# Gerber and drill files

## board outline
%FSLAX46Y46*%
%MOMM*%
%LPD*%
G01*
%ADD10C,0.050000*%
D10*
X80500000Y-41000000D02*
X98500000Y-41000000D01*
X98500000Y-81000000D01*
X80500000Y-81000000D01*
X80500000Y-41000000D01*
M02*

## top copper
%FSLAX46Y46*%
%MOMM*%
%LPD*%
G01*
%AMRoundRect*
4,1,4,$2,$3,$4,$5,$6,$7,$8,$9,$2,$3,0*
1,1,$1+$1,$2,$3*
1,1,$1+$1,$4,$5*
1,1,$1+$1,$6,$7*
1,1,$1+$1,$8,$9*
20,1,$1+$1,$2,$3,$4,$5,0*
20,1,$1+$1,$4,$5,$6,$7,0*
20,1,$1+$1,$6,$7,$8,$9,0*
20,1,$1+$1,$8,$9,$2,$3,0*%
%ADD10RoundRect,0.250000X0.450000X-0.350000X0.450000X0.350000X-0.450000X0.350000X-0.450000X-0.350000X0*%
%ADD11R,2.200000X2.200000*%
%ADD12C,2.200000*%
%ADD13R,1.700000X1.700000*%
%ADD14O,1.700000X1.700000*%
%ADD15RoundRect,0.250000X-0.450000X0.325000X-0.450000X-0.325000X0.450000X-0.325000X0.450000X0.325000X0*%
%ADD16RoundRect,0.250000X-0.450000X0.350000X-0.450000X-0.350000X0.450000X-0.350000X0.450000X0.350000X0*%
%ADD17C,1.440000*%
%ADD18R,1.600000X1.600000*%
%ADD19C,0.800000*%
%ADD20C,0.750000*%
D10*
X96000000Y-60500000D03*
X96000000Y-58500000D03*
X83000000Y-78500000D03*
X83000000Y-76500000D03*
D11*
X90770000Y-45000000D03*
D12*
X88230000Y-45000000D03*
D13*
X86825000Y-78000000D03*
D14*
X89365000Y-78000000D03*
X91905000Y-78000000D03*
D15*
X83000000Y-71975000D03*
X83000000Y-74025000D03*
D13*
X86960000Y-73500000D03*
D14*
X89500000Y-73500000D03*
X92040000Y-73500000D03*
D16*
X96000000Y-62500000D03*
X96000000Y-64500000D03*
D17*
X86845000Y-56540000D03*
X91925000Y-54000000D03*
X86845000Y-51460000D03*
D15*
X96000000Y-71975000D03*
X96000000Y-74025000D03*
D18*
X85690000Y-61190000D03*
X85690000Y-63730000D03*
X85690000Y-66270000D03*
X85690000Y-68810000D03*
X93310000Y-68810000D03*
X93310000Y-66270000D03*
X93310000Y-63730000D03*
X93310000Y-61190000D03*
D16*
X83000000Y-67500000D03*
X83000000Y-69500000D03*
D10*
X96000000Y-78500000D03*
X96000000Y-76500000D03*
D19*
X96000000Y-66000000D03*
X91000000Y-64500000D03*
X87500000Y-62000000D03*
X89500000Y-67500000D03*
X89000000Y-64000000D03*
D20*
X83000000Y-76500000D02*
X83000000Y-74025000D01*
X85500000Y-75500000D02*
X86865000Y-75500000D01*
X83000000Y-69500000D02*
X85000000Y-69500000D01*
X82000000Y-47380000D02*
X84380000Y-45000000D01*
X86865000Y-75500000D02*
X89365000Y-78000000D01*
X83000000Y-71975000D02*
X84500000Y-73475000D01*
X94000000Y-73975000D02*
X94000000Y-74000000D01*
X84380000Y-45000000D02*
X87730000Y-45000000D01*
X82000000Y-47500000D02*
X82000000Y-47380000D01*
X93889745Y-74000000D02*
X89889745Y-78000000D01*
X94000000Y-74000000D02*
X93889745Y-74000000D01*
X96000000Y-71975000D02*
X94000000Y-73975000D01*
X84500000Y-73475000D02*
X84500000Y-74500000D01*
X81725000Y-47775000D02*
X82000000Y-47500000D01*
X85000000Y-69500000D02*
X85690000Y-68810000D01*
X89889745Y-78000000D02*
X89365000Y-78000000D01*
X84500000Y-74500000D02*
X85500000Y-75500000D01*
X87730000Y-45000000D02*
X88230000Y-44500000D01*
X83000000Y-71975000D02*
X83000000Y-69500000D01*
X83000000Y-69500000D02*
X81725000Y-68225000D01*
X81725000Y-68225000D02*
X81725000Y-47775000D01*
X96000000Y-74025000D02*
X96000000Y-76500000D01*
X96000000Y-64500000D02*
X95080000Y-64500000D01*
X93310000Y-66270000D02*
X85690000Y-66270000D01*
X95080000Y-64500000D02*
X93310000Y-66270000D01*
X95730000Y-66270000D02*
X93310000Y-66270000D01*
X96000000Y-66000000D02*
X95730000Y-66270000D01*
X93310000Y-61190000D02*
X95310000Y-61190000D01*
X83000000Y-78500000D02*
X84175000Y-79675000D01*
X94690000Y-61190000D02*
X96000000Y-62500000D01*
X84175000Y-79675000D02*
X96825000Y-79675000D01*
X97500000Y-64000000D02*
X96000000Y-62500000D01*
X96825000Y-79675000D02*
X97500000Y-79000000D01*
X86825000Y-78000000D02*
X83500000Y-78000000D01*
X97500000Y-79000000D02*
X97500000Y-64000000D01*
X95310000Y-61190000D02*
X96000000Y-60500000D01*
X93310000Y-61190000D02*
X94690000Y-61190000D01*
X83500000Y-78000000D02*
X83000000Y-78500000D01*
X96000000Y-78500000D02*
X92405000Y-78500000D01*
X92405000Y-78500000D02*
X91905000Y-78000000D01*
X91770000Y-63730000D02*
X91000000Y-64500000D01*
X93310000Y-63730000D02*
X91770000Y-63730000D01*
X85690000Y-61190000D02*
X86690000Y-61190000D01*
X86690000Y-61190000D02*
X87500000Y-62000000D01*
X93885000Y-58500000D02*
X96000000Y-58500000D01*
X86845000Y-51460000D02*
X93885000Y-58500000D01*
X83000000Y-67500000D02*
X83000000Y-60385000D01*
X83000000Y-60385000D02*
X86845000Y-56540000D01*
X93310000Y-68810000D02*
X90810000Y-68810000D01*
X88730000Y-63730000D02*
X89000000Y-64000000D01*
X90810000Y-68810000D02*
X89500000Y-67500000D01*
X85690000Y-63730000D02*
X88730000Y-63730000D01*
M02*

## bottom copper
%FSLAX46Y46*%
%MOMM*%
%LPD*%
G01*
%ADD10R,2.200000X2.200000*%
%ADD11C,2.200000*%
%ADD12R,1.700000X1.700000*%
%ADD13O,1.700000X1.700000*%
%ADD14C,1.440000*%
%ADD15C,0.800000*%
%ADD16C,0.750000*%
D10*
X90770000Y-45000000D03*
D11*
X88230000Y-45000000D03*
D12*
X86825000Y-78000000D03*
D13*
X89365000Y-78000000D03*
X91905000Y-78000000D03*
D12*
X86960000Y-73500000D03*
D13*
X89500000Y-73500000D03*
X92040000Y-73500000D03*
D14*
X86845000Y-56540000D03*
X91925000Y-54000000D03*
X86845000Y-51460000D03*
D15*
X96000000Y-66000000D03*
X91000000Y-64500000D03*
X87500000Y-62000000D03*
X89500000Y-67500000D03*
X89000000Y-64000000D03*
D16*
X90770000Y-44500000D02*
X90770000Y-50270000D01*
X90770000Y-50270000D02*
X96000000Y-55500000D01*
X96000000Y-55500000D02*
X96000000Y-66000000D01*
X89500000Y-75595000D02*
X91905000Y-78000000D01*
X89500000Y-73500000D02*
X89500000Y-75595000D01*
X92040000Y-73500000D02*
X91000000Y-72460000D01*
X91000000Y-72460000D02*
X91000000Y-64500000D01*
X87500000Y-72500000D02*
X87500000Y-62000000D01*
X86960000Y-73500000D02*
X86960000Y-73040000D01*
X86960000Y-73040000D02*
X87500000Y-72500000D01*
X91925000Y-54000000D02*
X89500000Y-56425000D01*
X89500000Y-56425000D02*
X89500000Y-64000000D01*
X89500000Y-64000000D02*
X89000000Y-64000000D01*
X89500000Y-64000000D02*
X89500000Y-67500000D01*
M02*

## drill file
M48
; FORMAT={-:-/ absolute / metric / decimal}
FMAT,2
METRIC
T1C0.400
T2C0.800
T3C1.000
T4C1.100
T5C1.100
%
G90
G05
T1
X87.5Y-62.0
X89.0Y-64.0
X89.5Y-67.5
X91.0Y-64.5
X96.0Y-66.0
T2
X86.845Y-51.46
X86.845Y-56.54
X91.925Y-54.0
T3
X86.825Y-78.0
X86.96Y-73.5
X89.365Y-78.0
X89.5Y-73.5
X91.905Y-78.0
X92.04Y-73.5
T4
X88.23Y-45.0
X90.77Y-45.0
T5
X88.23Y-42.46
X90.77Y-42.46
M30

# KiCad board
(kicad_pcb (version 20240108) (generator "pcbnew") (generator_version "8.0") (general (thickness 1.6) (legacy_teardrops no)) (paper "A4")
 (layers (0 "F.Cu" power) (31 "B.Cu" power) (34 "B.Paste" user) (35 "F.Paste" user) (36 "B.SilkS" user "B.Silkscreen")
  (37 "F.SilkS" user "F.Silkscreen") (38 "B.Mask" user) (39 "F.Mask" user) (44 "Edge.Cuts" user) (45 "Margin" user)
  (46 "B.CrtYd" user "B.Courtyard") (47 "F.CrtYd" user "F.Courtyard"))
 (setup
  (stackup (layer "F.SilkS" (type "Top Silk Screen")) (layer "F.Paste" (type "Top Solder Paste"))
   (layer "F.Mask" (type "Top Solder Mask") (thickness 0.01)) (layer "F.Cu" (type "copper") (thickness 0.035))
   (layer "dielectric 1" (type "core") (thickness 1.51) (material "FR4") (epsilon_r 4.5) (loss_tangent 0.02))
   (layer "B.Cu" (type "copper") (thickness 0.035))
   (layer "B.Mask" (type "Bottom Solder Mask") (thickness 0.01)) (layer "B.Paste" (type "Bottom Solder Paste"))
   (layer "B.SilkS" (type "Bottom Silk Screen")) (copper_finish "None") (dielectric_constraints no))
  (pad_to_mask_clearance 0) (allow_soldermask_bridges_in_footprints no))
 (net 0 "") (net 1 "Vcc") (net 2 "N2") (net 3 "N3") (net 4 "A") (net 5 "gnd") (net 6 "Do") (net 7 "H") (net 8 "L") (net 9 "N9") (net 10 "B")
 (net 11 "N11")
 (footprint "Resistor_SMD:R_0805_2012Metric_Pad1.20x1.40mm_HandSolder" (layer "F.Cu") (at 96 59.5 90)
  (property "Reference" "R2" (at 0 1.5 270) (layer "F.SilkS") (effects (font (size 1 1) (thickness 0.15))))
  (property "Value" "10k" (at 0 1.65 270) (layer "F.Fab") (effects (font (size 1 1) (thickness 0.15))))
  (pad "1" smd roundrect (at -1 0 90) (size 1.2 1.4) (layers "F.Cu" "F.Paste" "F.Mask") (roundrect_rratio 0.208333) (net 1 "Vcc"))
  (pad "2" smd roundrect (at 1 0 90) (size 1.2 1.4) (layers "F.Cu" "F.Paste" "F.Mask") (roundrect_rratio 0.208333) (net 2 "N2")))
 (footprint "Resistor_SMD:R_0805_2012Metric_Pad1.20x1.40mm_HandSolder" (layer "F.Cu") (at 83 77.5 90)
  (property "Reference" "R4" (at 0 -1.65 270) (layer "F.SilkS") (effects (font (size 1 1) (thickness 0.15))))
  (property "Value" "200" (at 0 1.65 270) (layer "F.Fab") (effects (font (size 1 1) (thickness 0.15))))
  (pad "1" smd roundrect (at -1 0 90) (size 1.2 1.4) (layers "F.Cu" "F.Paste" "F.Mask") (roundrect_rratio 0.208333) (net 1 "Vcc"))
  (pad "2" smd roundrect (at 1 0 90) (size 1.2 1.4) (layers "F.Cu" "F.Paste" "F.Mask") (roundrect_rratio 0.208333) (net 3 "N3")))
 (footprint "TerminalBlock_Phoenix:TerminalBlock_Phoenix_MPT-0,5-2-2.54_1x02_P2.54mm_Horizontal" (layer "F.Cu") (at 90.77 45 180)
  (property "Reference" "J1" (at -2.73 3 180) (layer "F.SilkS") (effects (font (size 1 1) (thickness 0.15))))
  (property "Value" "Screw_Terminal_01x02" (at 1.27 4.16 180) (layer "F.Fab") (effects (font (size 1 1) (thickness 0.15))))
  (pad "" np_thru_hole circle (at 0 2.54 180) (size 1.1 1.1) (drill 1.1) (layers "*.Cu" "*.Mask"))
  (pad "" np_thru_hole circle (at 2.54 2.54 180) (size 1.1 1.1) (drill 1.1) (layers "*.Cu" "*.Mask"))
  (pad "1" thru_hole rect (at 0 0 180) (size 2.2 2.2) (drill 1.1) (layers "*.Cu" "*.Mask") (remove_unused_layers no) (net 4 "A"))
  (pad "2" thru_hole circle (at 2.54 0 180) (size 2.2 2.2) (drill 1.1) (layers "*.Cu" "*.Mask") (remove_unused_layers no) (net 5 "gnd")))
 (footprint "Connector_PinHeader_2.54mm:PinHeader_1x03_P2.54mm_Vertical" (layer "F.Cu") (at 86.825 78 90)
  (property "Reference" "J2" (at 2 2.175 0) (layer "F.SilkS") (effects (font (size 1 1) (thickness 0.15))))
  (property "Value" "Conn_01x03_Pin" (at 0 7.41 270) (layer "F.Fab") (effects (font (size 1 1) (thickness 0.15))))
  (pad "1" thru_hole rect (at 0 0 90) (size 1.7 1.7) (drill 1) (layers "*.Cu" "*.Mask") (remove_unused_layers no) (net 1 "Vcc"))
  (pad "2" thru_hole oval (at 0 2.54 90) (size 1.7 1.7) (drill 1) (layers "*.Cu" "*.Mask") (remove_unused_layers no) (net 5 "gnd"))
  (pad "3" thru_hole oval (at 0 5.08 90) (size 1.7 1.7) (drill 1) (layers "*.Cu" "*.Mask") (remove_unused_layers no) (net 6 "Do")))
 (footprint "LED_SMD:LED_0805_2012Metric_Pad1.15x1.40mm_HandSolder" (layer "F.Cu") (at 83 73 -90)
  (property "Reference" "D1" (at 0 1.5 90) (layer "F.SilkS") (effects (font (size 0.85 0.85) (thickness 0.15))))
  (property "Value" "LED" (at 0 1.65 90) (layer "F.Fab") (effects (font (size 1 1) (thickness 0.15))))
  (pad "1" smd roundrect (at -1.025 0 270) (size 1.15 1.4) (layers "F.Cu" "F.Paste" "F.Mask") (roundrect_rratio 0.217391) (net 5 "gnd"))
  (pad "2" smd roundrect (at 1.025 0 270) (size 1.15 1.4) (layers "F.Cu" "F.Paste" "F.Mask") (roundrect_rratio 0.217391) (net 3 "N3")))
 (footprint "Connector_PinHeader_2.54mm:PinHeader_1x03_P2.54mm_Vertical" (layer "F.Cu") (at 86.96 73.5 90)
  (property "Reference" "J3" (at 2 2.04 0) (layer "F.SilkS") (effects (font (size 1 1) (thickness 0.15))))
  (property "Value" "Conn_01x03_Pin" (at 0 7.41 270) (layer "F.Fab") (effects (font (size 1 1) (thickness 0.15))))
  (pad "1" thru_hole rect (at 0 0 90) (size 1.7 1.7) (drill 1) (layers "*.Cu" "*.Mask") (remove_unused_layers no) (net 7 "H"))
  (pad "2" thru_hole oval (at 0 2.54 90) (size 1.7 1.7) (drill 1) (layers "*.Cu" "*.Mask") (remove_unused_layers no) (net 6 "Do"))
  (pad "3" thru_hole oval (at 0 5.08 90) (size 1.7 1.7) (drill 1) (layers "*.Cu" "*.Mask") (remove_unused_layers no) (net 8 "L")))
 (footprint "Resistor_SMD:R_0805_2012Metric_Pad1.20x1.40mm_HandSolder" (layer "F.Cu") (at 96 63.5 -90)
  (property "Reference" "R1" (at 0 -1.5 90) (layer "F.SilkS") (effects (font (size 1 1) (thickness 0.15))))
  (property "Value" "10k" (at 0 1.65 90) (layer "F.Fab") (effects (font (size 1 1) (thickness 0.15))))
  (pad "1" smd roundrect (at -1 0 270) (size 1.2 1.4) (layers "F.Cu" "F.Paste" "F.Mask") (roundrect_rratio 0.208333) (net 1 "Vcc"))
  (pad "2" smd roundrect (at 1 0 270) (size 1.2 1.4) (layers "F.Cu" "F.Paste" "F.Mask") (roundrect_rratio 0.208333) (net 4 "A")))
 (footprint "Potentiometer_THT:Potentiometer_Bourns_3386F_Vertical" (layer "F.Cu") (at 86.845 56.54)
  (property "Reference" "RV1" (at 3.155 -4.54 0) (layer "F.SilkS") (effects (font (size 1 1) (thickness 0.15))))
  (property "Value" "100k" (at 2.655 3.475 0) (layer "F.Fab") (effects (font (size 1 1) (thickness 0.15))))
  (pad "1" thru_hole circle (at 0 0) (size 1.44 1.44) (drill 0.8) (layers "*.Cu" "*.Mask") (remove_unused_layers no) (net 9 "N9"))
  (pad "2" thru_hole circle (at 5.08 -2.54) (size 1.44 1.44) (drill 0.8) (layers "*.Cu" "*.Mask") (remove_unused_layers no) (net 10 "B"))
  (pad "3" thru_hole circle (at 0 -5.08) (size 1.44 1.44) (drill 0.8) (layers "*.Cu" "*.Mask") (remove_unused_layers no) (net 2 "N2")))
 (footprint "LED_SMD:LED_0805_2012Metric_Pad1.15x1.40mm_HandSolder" (layer "F.Cu") (at 96 73 -90)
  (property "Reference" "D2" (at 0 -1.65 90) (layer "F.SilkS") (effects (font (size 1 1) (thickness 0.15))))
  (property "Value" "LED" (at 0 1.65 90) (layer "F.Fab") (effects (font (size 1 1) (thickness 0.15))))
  (pad "1" smd roundrect (at -1.025 0 270) (size 1.15 1.4) (layers "F.Cu" "F.Paste" "F.Mask") (roundrect_rratio 0.217391) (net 5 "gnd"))
  (pad "2" smd roundrect (at 1.025 0 270) (size 1.15 1.4) (layers "F.Cu" "F.Paste" "F.Mask") (roundrect_rratio 0.217391) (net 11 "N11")))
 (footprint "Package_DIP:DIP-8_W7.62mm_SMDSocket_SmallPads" (layer "F.Cu") (at 89.5 65)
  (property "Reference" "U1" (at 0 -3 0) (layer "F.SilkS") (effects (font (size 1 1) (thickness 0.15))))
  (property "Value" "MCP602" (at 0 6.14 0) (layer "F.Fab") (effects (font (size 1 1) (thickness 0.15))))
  (pad "1" smd rect (at -3.81 -3.81) (size 1.6 1.6) (layers "F.Cu" "F.Paste" "F.Mask") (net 7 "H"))
  (pad "2" smd rect (at -3.81 -1.27) (size 1.6 1.6) (layers "F.Cu" "F.Paste" "F.Mask") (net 10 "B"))
  (pad "3" smd rect (at -3.81 1.27) (size 1.6 1.6) (layers "F.Cu" "F.Paste" "F.Mask") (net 4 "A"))
  (pad "4" smd rect (at -3.81 3.81) (size 1.6 1.6) (layers "F.Cu" "F.Paste" "F.Mask") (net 5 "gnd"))
  (pad "5" smd rect (at 3.81 3.81) (size 1.6 1.6) (layers "F.Cu" "F.Paste" "F.Mask") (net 10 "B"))
  (pad "6" smd rect (at 3.81 1.27) (size 1.6 1.6) (layers "F.Cu" "F.Paste" "F.Mask") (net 4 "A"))
  (pad "7" smd rect (at 3.81 -1.27) (size 1.6 1.6) (layers "F.Cu" "F.Paste" "F.Mask") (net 8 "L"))
  (pad "8" smd rect (at 3.81 -3.81) (size 1.6 1.6) (layers "F.Cu" "F.Paste" "F.Mask") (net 1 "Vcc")))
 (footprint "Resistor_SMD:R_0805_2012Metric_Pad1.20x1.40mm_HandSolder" (layer "F.Cu") (at 83 68.5 -90)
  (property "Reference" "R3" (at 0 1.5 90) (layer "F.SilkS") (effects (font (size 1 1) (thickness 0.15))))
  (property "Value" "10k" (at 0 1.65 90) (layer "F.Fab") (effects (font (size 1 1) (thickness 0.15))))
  (pad "1" smd roundrect (at -1 0 270) (size 1.2 1.4) (layers "F.Cu" "F.Paste" "F.Mask") (roundrect_rratio 0.208333) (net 9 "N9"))
  (pad "2" smd roundrect (at 1 0 270) (size 1.2 1.4) (layers "F.Cu" "F.Paste" "F.Mask") (roundrect_rratio 0.208333) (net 5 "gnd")))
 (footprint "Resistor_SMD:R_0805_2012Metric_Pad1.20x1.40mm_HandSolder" (layer "F.Cu") (at 96 77.5 90)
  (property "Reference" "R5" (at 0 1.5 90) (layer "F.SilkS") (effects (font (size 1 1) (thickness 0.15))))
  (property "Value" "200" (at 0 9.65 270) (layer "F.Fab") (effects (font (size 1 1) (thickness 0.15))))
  (pad "1" smd roundrect (at -1 0 90) (size 1.2 1.4) (layers "F.Cu" "F.Paste" "F.Mask") (roundrect_rratio 0.208333) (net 6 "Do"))
  (pad "2" smd roundrect (at 1 0 90) (size 1.2 1.4) (layers "F.Cu" "F.Paste" "F.Mask") (roundrect_rratio 0.208333) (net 11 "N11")))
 (gr_rect (start 80.5 41) (end 98.5 81) (stroke (width 0.05) (type default)) (fill none) (layer "Edge.Cuts"))
 (segment (start 83 76.5) (end 83 74.025) (width 0.75) (layer "F.Cu") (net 3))
 (segment (start 85.5 75.5) (end 86.865 75.5) (width 0.75) (layer "F.Cu") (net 5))
 (segment (start 83 69.5) (end 85 69.5) (width 0.75) (layer "F.Cu") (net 5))
 (segment (start 82 47.38) (end 84.38 45) (width 0.75) (layer "F.Cu") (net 5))
 (segment (start 86.865 75.5) (end 89.365 78) (width 0.75) (layer "F.Cu") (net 5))
 (segment (start 83 71.975) (end 84.5 73.475) (width 0.75) (layer "F.Cu") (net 5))
 (segment (start 94 73.975) (end 94 74) (width 0.75) (layer "F.Cu") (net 5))
 (segment (start 84.38 45) (end 87.73 45) (width 0.75) (layer "F.Cu") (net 5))
 (segment (start 82 47.5) (end 82 47.38) (width 0.75) (layer "F.Cu") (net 5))
 (segment (start 93.889745 74) (end 89.889745 78) (width 0.75) (layer "F.Cu") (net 5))
 (segment (start 94 74) (end 93.889745 74) (width 0.75) (layer "F.Cu") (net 5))
 (segment (start 96 71.975) (end 94 73.975) (width 0.75) (layer "F.Cu") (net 5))
 (segment (start 84.5 73.475) (end 84.5 74.5) (width 0.75) (layer "F.Cu") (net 5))
 (segment (start 81.725 47.775) (end 82 47.5) (width 0.75) (layer "F.Cu") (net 5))
 (segment (start 85 69.5) (end 85.69 68.81) (width 0.75) (layer "F.Cu") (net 5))
 (segment (start 89.889745 78) (end 89.365 78) (width 0.75) (layer "F.Cu") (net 5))
 (segment (start 84.5 74.5) (end 85.5 75.5) (width 0.75) (layer "F.Cu") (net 5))
 (segment (start 87.73 45) (end 88.23 44.5) (width 0.75) (layer "F.Cu") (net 5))
 (segment (start 83 71.975) (end 83 69.5) (width 0.75) (layer "F.Cu") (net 5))
 (segment (start 83 69.5) (end 81.725 68.225) (width 0.75) (layer "F.Cu") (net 5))
 (segment (start 81.725 68.225) (end 81.725 47.775) (width 0.75) (layer "F.Cu") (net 5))
 (segment (start 96 74.025) (end 96 76.5) (width 0.75) (layer "F.Cu") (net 11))
 (segment (start 96 64.5) (end 95.08 64.5) (width 0.75) (layer "F.Cu") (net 4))
 (segment (start 93.31 66.27) (end 85.69 66.27) (width 0.75) (layer "F.Cu") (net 4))
 (segment (start 95.08 64.5) (end 93.31 66.27) (width 0.75) (layer "F.Cu") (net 4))
 (segment (start 95.73 66.27) (end 93.31 66.27) (width 0.75) (layer "F.Cu") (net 4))
 (segment (start 96 66) (end 95.73 66.27) (width 0.75) (layer "F.Cu") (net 4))
 (via (at 96 66) (size 0.8) (drill 0.4) (layers "F.Cu" "B.Cu") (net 4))
 (segment (start 90.77 44.5) (end 90.77 50.27) (width 0.75) (layer "B.Cu") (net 4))
 (segment (start 90.77 50.27) (end 96 55.5) (width 0.75) (layer "B.Cu") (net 4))
 (segment (start 96 55.5) (end 96 66) (width 0.75) (layer "B.Cu") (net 4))
 (segment (start 93.31 61.19) (end 95.31 61.19) (width 0.75) (layer "F.Cu") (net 1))
 (segment (start 83 78.5) (end 84.175 79.675) (width 0.75) (layer "F.Cu") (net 1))
 (segment (start 94.69 61.19) (end 96 62.5) (width 0.75) (layer "F.Cu") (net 1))
 (segment (start 84.175 79.675) (end 96.825 79.675) (width 0.75) (layer "F.Cu") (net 1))
 (segment (start 97.5 64) (end 96 62.5) (width 0.75) (layer "F.Cu") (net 1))
 (segment (start 96.825 79.675) (end 97.5 79) (width 0.75) (layer "F.Cu") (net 1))
 (segment (start 86.825 78) (end 83.5 78) (width 0.75) (layer "F.Cu") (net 1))
 (segment (start 97.5 79) (end 97.5 64) (width 0.75) (layer "F.Cu") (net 1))
 (segment (start 95.31 61.19) (end 96 60.5) (width 0.75) (layer "F.Cu") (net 1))
 (segment (start 93.31 61.19) (end 94.69 61.19) (width 0.75) (layer "F.Cu") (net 1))
 (segment (start 83.5 78) (end 83 78.5) (width 0.75) (layer "F.Cu") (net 1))
 (segment (start 96 78.5) (end 92.405 78.5) (width 0.75) (layer "F.Cu") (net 6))
 (segment (start 92.405 78.5) (end 91.905 78) (width 0.75) (layer "F.Cu") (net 6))
 (segment (start 89.5 75.595) (end 91.905 78) (width 0.75) (layer "B.Cu") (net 6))
 (segment (start 89.5 73.5) (end 89.5 75.595) (width 0.75) (layer "B.Cu") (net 6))
 (segment (start 91.77 63.73) (end 91 64.5) (width 0.75) (layer "F.Cu") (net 8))
 (segment (start 93.31 63.73) (end 91.77 63.73) (width 0.75) (layer "F.Cu") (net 8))
 (via (at 91 64.5) (size 0.8) (drill 0.4) (layers "F.Cu" "B.Cu") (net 8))
 (segment (start 92.04 73.5) (end 91 72.46) (width 0.75) (layer "B.Cu") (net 8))
 (segment (start 91 72.46) (end 91 64.5) (width 0.75) (layer "B.Cu") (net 8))
 (segment (start 85.69 61.19) (end 86.69 61.19) (width 0.75) (layer "F.Cu") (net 7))
 (segment (start 86.69 61.19) (end 87.5 62) (width 0.75) (layer "F.Cu") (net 7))
 (via (at 87.5 62) (size 0.8) (drill 0.4) (layers "F.Cu" "B.Cu") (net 7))
 (segment (start 87.5 72.5) (end 87.5 62) (width 0.75) (layer "B.Cu") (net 7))
 (segment (start 86.96 73.5) (end 86.96 73.04) (width 0.75) (layer "B.Cu") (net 7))
 (segment (start 86.96 73.04) (end 87.5 72.5) (width 0.75) (layer "B.Cu") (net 7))
 (segment (start 93.885 58.5) (end 96 58.5) (width 0.75) (layer "F.Cu") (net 2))
 (segment (start 86.845 51.46) (end 93.885 58.5) (width 0.75) (layer "F.Cu") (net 2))
 (segment (start 83 67.5) (end 83 60.385) (width 0.75) (layer "F.Cu") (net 9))
 (segment (start 83 60.385) (end 86.845 56.54) (width 0.75) (layer "F.Cu") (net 9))
 (segment (start 93.31 68.81) (end 90.81 68.81) (width 0.75) (layer "F.Cu") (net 10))
 (segment (start 88.73 63.73) (end 89 64) (width 0.75) (layer "F.Cu") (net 10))
 (segment (start 90.81 68.81) (end 89.5 67.5) (width 0.75) (layer "F.Cu") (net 10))
 (segment (start 85.69 63.73) (end 88.73 63.73) (width 0.75) (layer "F.Cu") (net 10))
 (via (at 89.5 67.5) (size 0.8) (drill 0.4) (layers "F.Cu" "B.Cu") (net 10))
 (via (at 89 64) (size 0.8) (drill 0.4) (layers "F.Cu" "B.Cu") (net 10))
 (segment (start 91.925 54) (end 89.5 56.425) (width 0.75) (layer "B.Cu") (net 10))
 (segment (start 89.5 56.425) (end 89.5 64) (width 0.75) (layer "B.Cu") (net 10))
 (segment (start 89.5 64) (end 89 64) (width 0.75) (layer "B.Cu") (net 10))
 (segment (start 89.5 64) (end 89.5 67.5) (width 0.75) (layer "B.Cu") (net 10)))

